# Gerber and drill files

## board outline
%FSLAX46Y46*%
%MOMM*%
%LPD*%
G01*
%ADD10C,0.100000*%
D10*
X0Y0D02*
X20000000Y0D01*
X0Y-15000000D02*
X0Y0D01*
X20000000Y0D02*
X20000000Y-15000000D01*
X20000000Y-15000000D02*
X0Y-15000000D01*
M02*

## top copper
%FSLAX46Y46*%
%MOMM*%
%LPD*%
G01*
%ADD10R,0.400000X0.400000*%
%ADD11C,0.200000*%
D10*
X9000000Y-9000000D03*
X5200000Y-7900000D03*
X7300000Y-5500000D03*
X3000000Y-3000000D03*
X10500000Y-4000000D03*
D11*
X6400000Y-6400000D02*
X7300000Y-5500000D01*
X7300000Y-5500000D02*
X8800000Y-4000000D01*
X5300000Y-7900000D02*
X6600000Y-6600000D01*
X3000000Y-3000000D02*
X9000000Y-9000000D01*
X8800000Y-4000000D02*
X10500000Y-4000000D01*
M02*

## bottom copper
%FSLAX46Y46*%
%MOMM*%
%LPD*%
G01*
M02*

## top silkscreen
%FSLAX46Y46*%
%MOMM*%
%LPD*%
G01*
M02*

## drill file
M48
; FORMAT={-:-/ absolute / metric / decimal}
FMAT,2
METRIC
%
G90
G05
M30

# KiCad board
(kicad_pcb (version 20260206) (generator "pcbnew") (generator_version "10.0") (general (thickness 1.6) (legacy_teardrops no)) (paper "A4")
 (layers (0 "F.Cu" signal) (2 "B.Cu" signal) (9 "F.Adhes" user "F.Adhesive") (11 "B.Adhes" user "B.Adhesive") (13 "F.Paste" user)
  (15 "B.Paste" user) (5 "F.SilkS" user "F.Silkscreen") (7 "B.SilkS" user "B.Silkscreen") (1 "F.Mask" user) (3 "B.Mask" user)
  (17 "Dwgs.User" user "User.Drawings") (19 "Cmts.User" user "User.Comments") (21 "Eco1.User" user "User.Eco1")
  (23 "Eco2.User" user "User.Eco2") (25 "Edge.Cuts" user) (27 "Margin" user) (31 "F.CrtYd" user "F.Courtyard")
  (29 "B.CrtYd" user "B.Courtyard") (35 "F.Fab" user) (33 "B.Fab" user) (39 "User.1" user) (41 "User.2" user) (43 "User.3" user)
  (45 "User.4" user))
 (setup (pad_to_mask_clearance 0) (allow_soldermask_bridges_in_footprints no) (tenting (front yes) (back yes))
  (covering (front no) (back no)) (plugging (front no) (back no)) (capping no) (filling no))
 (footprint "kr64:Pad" (layer "F.Cu") (at 9 9)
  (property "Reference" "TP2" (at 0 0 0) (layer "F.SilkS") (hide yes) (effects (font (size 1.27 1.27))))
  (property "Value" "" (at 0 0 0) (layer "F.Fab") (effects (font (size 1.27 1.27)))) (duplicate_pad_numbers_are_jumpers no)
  (pad "1" smd rect (at 0 0) (size 0.4 0.4) (layers "F.Cu" "F.Mask" "F.Paste") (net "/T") (thermal_bridge_angle 45)))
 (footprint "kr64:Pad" (layer "F.Cu") (at 5.2 7.9)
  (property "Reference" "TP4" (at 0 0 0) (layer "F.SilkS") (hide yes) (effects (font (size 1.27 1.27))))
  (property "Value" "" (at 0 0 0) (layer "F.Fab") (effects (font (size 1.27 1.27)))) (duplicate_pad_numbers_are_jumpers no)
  (pad "1" smd rect (at 0 0) (size 0.4 0.4) (layers "F.Cu" "F.Mask" "F.Paste") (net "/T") (thermal_bridge_angle 45)))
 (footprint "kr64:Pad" (layer "F.Cu") (at 7.3 5.5)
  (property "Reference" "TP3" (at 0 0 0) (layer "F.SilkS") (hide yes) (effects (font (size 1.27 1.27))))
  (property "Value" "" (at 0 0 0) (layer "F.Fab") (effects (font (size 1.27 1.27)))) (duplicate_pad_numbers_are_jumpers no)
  (pad "1" smd rect (at 0 0) (size 0.4 0.4) (layers "F.Cu" "F.Mask" "F.Paste") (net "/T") (thermal_bridge_angle 45)))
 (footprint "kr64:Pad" (layer "F.Cu") (at 3 3)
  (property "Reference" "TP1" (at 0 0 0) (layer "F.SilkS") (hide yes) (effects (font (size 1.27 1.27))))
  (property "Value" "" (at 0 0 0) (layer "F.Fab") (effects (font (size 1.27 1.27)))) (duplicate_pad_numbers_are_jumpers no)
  (pad "1" smd rect (at 0 0) (size 0.4 0.4) (layers "F.Cu" "F.Mask" "F.Paste") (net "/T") (thermal_bridge_angle 45)))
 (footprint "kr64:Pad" (layer "F.Cu") (at 10.5 4)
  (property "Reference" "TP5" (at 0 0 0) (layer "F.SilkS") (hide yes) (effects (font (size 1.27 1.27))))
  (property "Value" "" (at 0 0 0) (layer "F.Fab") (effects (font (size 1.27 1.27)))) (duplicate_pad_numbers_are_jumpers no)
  (pad "1" smd rect (at 0 0) (size 0.4 0.4) (layers "F.Cu" "F.Mask" "F.Paste") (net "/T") (thermal_bridge_angle 45)))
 (gr_line (start 0 0) (end 20 0) (stroke (width 0.1) (type default)) (layer "Edge.Cuts"))
 (gr_line (start 0 15) (end 0 0) (stroke (width 0.1) (type default)) (layer "Edge.Cuts"))
 (gr_line (start 20 0) (end 20 15) (stroke (width 0.1) (type default)) (layer "Edge.Cuts"))
 (gr_line (start 20 15) (end 0 15) (stroke (width 0.1) (type default)) (layer "Edge.Cuts"))
 (segment (start 6.4 6.4) (end 7.3 5.5) (width 0.2) (layer "F.Cu") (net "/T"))
 (segment (start 7.3 5.5) (end 8.8 4) (width 0.2) (layer "F.Cu") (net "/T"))
 (segment (start 5.3 7.9) (end 6.6 6.6) (width 0.2) (layer "F.Cu") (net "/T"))
 (segment (start 3 3) (end 9 9) (width 0.2) (layer "F.Cu") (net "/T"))
 (segment (start 8.8 4) (end 10.5 4) (width 0.2) (layer "F.Cu") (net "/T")))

